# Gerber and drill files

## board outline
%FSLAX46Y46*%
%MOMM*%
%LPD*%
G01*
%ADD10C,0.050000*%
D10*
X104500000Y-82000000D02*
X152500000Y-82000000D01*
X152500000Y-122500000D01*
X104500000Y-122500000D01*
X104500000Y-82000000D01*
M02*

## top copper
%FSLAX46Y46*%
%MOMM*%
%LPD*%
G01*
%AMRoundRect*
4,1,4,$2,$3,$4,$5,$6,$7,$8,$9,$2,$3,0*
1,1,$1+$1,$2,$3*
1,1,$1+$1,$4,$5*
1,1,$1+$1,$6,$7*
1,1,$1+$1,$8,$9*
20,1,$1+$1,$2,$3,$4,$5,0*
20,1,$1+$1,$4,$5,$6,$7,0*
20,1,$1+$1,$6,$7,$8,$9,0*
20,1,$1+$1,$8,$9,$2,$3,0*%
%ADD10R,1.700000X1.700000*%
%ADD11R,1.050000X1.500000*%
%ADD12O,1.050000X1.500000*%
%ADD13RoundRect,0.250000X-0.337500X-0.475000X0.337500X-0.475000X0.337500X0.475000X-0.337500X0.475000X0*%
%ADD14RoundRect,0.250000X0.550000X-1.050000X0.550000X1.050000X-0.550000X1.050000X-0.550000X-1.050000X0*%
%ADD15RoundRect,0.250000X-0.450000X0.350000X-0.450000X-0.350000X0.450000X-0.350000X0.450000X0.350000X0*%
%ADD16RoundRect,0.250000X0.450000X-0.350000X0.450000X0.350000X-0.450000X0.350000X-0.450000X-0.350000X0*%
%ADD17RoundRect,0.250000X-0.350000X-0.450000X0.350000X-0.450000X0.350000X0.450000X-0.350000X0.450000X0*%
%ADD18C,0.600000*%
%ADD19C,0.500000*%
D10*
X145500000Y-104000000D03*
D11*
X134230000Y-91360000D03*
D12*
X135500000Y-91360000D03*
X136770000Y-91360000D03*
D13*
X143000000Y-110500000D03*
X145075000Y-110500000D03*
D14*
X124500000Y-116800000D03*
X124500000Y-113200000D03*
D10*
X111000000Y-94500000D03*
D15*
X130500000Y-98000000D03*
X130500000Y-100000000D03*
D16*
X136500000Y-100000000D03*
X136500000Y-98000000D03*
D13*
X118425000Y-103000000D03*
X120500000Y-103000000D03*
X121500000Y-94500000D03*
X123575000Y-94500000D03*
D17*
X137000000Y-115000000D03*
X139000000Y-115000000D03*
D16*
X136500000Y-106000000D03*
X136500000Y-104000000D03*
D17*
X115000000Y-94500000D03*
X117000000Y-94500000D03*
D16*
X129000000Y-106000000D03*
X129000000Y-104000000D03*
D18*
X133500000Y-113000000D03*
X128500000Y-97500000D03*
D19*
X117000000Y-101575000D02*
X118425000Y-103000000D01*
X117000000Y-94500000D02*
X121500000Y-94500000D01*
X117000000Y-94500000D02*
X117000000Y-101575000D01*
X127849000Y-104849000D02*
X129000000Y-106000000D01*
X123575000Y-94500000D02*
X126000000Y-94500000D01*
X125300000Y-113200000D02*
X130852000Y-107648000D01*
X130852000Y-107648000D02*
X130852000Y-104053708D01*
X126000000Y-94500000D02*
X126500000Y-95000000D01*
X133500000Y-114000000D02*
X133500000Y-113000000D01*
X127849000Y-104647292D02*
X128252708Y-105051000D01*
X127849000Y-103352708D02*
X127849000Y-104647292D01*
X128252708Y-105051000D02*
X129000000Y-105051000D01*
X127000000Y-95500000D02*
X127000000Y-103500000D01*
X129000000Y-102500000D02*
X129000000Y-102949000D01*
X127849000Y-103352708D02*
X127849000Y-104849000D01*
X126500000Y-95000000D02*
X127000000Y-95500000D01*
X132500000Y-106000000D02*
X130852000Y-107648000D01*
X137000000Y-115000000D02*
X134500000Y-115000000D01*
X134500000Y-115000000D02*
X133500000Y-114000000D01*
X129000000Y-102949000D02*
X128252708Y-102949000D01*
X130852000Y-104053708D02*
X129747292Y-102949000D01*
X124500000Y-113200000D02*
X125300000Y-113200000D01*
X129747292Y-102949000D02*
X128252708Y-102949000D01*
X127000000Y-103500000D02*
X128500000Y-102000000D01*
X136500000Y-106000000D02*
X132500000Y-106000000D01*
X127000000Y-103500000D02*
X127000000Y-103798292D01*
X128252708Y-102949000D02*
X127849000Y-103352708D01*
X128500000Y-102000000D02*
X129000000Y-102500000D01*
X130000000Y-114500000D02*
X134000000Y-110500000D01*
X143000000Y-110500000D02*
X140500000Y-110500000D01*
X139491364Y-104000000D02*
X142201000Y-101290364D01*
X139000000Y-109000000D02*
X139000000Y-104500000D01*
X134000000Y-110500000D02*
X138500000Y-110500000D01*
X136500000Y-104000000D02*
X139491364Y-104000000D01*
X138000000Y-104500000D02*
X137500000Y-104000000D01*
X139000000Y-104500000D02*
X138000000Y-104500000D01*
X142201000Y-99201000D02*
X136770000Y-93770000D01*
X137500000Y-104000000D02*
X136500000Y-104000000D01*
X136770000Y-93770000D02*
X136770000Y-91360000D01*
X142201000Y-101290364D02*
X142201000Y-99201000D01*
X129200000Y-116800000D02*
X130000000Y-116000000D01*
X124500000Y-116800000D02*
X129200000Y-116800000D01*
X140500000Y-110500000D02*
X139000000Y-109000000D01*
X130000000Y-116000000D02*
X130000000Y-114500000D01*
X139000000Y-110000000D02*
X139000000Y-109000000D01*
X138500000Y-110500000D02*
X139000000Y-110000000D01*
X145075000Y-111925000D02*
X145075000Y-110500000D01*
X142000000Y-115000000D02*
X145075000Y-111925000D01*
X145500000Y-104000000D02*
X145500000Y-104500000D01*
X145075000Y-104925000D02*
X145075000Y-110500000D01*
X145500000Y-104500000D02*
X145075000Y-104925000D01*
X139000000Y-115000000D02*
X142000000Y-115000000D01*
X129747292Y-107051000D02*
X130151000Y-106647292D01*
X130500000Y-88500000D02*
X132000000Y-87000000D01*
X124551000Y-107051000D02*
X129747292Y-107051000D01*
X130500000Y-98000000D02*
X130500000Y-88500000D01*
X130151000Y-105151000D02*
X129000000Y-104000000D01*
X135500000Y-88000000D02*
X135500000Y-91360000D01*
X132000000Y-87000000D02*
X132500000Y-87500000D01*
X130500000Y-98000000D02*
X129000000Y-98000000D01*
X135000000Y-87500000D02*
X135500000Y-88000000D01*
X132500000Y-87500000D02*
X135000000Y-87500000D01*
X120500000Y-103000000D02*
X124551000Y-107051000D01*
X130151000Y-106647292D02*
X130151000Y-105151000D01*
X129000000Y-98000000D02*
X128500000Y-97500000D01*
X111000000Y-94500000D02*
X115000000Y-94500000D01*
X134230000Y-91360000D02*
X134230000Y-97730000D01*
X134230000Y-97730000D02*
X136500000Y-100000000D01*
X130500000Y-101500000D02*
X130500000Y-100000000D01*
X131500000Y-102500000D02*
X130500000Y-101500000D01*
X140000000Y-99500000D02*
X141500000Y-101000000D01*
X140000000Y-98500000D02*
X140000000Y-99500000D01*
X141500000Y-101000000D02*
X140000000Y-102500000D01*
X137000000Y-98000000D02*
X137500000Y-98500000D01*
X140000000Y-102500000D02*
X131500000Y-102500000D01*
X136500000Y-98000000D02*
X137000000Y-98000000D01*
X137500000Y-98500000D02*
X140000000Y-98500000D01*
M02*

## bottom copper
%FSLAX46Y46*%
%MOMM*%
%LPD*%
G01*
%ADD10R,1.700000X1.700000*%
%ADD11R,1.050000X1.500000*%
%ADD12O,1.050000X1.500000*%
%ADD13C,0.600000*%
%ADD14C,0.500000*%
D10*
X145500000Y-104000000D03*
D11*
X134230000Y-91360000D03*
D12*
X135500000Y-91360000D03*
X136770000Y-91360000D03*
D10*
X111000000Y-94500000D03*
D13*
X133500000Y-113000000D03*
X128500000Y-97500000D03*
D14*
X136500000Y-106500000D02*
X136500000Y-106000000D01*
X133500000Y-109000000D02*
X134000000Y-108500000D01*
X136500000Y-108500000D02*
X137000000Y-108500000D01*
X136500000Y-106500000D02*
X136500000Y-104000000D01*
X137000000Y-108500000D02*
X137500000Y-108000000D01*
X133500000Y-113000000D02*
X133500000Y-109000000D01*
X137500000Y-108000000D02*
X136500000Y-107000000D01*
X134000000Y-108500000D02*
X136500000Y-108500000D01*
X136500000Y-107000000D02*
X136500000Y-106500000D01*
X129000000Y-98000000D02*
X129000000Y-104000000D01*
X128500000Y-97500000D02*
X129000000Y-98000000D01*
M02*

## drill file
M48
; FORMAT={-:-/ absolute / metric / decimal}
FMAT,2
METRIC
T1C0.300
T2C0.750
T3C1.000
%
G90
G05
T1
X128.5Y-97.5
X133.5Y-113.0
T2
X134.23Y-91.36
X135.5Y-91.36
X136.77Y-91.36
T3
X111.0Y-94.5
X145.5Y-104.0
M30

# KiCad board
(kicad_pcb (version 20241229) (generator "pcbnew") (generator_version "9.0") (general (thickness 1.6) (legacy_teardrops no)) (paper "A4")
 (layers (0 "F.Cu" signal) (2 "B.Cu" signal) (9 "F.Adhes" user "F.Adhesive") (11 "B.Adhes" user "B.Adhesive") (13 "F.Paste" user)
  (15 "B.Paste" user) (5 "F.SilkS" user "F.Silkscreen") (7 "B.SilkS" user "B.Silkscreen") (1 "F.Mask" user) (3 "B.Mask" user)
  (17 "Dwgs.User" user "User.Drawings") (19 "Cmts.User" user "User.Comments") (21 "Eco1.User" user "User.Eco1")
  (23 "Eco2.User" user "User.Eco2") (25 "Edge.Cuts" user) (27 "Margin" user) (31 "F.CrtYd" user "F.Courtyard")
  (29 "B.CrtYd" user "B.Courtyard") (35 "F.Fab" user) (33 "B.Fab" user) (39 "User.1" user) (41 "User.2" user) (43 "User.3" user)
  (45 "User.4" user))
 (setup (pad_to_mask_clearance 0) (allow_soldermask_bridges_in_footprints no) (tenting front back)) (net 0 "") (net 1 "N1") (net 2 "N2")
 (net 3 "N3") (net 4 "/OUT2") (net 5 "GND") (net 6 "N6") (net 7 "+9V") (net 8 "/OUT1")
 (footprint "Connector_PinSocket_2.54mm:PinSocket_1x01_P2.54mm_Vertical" (layer "F.Cu") (at 145.5 104)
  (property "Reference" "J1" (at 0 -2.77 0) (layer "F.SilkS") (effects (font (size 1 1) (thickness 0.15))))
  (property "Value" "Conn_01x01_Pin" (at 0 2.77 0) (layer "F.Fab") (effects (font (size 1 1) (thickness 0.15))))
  (pad "1" thru_hole rect (at 0 0) (size 1.7 1.7) (drill 1) (layers "*.Cu" "*.Mask") (remove_unused_layers no) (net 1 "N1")))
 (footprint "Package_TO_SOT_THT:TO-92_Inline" (layer "F.Cu") (at 134.23 91.36)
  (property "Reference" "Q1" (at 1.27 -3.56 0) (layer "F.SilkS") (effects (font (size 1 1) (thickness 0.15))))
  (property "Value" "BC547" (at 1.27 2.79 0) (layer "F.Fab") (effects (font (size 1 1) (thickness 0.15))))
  (pad "1" thru_hole rect (at 0 0) (size 1.05 1.5) (drill 0.75) (layers "*.Cu" "*.Mask") (remove_unused_layers no) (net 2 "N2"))
  (pad "2" thru_hole oval (at 1.27 0) (size 1.05 1.5) (drill 0.75) (layers "*.Cu" "*.Mask") (remove_unused_layers no) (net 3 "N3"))
  (pad "3" thru_hole oval (at 2.54 0) (size 1.05 1.5) (drill 0.75) (layers "*.Cu" "*.Mask") (remove_unused_layers no) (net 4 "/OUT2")))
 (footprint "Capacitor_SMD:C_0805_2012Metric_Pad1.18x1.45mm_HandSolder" (layer "F.Cu") (at 144.0375 110.5)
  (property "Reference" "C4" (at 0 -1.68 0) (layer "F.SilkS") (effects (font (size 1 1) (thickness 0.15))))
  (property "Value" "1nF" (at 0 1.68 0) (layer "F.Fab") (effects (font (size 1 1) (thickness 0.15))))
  (pad "1" smd roundrect (at -1.0375 0) (size 1.175 1.45) (layers "F.Cu" "F.Mask" "F.Paste") (roundrect_rratio 0.212766) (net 4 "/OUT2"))
  (pad "2" smd roundrect (at 1.0375 0) (size 1.175 1.45) (layers "F.Cu" "F.Mask" "F.Paste") (roundrect_rratio 0.212766) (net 1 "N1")))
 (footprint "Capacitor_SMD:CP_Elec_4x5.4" (layer "F.Cu") (at 124.5 115 90)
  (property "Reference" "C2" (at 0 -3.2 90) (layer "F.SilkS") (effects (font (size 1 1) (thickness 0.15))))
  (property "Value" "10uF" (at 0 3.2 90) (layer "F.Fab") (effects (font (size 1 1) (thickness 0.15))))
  (pad "1" smd roundrect (at -1.8 0 90) (size 2.6 1.6) (layers "F.Cu" "F.Mask" "F.Paste") (roundrect_rratio 0.15625) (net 4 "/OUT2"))
  (pad "2" smd roundrect (at 1.8 0 90) (size 2.6 1.6) (layers "F.Cu" "F.Mask" "F.Paste") (roundrect_rratio 0.15625) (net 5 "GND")))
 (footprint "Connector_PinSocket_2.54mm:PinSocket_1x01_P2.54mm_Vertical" (layer "F.Cu") (at 111 94.5)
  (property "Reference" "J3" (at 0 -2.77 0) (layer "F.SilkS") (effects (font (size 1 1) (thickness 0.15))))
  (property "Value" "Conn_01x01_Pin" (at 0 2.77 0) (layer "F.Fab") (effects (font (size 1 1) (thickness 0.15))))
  (pad "1" thru_hole rect (at 0 0) (size 1.7 1.7) (drill 1) (layers "*.Cu" "*.Mask") (remove_unused_layers no) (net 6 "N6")))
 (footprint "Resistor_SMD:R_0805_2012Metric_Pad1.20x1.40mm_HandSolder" (layer "F.Cu") (at 130.5 99 -90)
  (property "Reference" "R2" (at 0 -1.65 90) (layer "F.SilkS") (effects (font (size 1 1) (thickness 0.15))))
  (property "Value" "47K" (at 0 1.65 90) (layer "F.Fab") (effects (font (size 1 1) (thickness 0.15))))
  (pad "1" smd roundrect (at -1 0 270) (size 1.2 1.4) (layers "F.Cu" "F.Mask" "F.Paste") (roundrect_rratio 0.208333) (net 3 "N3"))
  (pad "2" smd roundrect (at 1 0 270) (size 1.2 1.4) (layers "F.Cu" "F.Mask" "F.Paste") (roundrect_rratio 0.208333) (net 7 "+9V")))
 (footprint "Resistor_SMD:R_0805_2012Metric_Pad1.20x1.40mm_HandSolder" (layer "F.Cu") (at 136.5 99 90)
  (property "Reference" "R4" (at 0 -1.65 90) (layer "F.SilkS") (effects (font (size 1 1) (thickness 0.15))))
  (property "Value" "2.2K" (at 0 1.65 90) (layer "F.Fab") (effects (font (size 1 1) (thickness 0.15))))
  (pad "1" smd roundrect (at -1 0 90) (size 1.2 1.4) (layers "F.Cu" "F.Mask" "F.Paste") (roundrect_rratio 0.208333) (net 2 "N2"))
  (pad "2" smd roundrect (at 1 0 90) (size 1.2 1.4) (layers "F.Cu" "F.Mask" "F.Paste") (roundrect_rratio 0.208333) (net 7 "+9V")))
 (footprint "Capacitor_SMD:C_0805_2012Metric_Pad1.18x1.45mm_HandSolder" (layer "F.Cu") (at 119.4625 103)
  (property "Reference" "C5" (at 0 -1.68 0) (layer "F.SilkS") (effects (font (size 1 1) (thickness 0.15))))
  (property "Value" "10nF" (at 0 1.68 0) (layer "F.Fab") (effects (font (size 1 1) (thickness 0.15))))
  (pad "1" smd roundrect (at -1.0375 0) (size 1.175 1.45) (layers "F.Cu" "F.Mask" "F.Paste") (roundrect_rratio 0.212766) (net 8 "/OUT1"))
  (pad "2" smd roundrect (at 1.0375 0) (size 1.175 1.45) (layers "F.Cu" "F.Mask" "F.Paste") (roundrect_rratio 0.212766) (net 3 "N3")))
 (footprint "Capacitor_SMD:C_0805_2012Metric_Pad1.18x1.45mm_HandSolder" (layer "F.Cu") (at 122.5375 94.5)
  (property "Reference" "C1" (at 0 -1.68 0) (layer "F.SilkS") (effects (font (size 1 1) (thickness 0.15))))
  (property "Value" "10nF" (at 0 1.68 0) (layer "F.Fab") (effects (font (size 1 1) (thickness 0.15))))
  (pad "1" smd roundrect (at -1.0375 0) (size 1.175 1.45) (layers "F.Cu" "F.Mask" "F.Paste") (roundrect_rratio 0.212766) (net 8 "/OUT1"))
  (pad "2" smd roundrect (at 1.0375 0) (size 1.175 1.45) (layers "F.Cu" "F.Mask" "F.Paste") (roundrect_rratio 0.212766) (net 5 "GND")))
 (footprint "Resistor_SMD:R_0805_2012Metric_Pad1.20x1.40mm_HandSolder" (layer "F.Cu") (at 138 115)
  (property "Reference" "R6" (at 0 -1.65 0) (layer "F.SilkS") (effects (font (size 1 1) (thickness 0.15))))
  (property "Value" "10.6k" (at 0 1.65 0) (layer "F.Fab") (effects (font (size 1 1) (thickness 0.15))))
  (pad "1" smd roundrect (at -1 0) (size 1.2 1.4) (layers "F.Cu" "F.Mask" "F.Paste") (roundrect_rratio 0.208333) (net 5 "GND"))
  (pad "2" smd roundrect (at 1 0) (size 1.2 1.4) (layers "F.Cu" "F.Mask" "F.Paste") (roundrect_rratio 0.208333) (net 1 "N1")))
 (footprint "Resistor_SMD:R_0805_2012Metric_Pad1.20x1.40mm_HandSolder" (layer "F.Cu") (at 136.5 105 90)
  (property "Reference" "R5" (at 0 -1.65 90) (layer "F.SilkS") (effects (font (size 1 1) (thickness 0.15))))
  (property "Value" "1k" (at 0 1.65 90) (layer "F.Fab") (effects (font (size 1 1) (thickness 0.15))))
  (pad "1" smd roundrect (at -1 0 90) (size 1.2 1.4) (layers "F.Cu" "F.Mask" "F.Paste") (roundrect_rratio 0.208333) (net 5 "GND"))
  (pad "2" smd roundrect (at 1 0 90) (size 1.2 1.4) (layers "F.Cu" "F.Mask" "F.Paste") (roundrect_rratio 0.208333) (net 4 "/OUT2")))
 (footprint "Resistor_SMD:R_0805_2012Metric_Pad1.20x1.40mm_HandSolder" (layer "F.Cu") (at 116 94.5)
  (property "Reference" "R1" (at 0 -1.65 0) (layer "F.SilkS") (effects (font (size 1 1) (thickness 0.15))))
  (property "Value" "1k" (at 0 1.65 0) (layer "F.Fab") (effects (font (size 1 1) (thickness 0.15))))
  (pad "1" smd roundrect (at -1 0) (size 1.2 1.4) (layers "F.Cu" "F.Mask" "F.Paste") (roundrect_rratio 0.208333) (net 6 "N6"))
  (pad "2" smd roundrect (at 1 0) (size 1.2 1.4) (layers "F.Cu" "F.Mask" "F.Paste") (roundrect_rratio 0.208333) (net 8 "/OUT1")))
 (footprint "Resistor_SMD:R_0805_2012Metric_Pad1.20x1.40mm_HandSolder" (layer "F.Cu") (at 129 105 90)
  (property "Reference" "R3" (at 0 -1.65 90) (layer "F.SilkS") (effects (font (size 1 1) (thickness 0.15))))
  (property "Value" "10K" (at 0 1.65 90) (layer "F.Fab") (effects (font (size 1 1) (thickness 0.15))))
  (pad "1" smd roundrect (at -1 0 90) (size 1.2 1.4) (layers "F.Cu" "F.Mask" "F.Paste") (roundrect_rratio 0.208333) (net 5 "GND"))
  (pad "2" smd roundrect (at 1 0 90) (size 1.2 1.4) (layers "F.Cu" "F.Mask" "F.Paste") (roundrect_rratio 0.208333) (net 3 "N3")))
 (gr_rect (start 104.5 82) (end 152.5 122.5) (stroke (width 0.05) (type default)) (fill no) (layer "Edge.Cuts"))
 (segment (start 117 101.575) (end 118.425 103) (width 0.5) (layer "F.Cu") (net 8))
 (segment (start 117 94.5) (end 121.5 94.5) (width 0.5) (layer "F.Cu") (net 8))
 (segment (start 117 94.5) (end 117 101.575) (width 0.5) (layer "F.Cu") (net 8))
 (segment (start 127.849 104.849) (end 129 106) (width 0.5) (layer "F.Cu") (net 5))
 (segment (start 123.575 94.5) (end 126 94.5) (width 0.5) (layer "F.Cu") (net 5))
 (segment (start 125.3 113.2) (end 130.852 107.648) (width 0.5) (layer "F.Cu") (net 5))
 (segment (start 130.852 107.648) (end 130.852 104.053708) (width 0.5) (layer "F.Cu") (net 5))
 (segment (start 126 94.5) (end 126.5 95) (width 0.5) (layer "F.Cu") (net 5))
 (segment (start 133.5 114) (end 133.5 113) (width 0.5) (layer "F.Cu") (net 5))
 (segment (start 127.849 104.647292) (end 128.252708 105.051) (width 0.5) (layer "F.Cu") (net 5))
 (segment (start 127.849 103.352708) (end 127.849 104.647292) (width 0.5) (layer "F.Cu") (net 5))
 (segment (start 128.252708 105.051) (end 129 105.051) (width 0.5) (layer "F.Cu") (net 5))
 (segment (start 127 95.5) (end 127 103.5) (width 0.5) (layer "F.Cu") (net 5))
 (segment (start 129 102.5) (end 129 102.949) (width 0.5) (layer "F.Cu") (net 5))
 (segment (start 127.849 103.352708) (end 127.849 104.849) (width 0.5) (layer "F.Cu") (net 5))
 (segment (start 126.5 95) (end 127 95.5) (width 0.5) (layer "F.Cu") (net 5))
 (segment (start 132.5 106) (end 130.852 107.648) (width 0.5) (layer "F.Cu") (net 5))
 (segment (start 137 115) (end 134.5 115) (width 0.5) (layer "F.Cu") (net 5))
 (segment (start 134.5 115) (end 133.5 114) (width 0.5) (layer "F.Cu") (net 5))
 (segment (start 129 102.949) (end 128.252708 102.949) (width 0.5) (layer "F.Cu") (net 5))
 (segment (start 130.852 104.053708) (end 129.747292 102.949) (width 0.5) (layer "F.Cu") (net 5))
 (segment (start 124.5 113.2) (end 125.3 113.2) (width 0.5) (layer "F.Cu") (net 5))
 (segment (start 129.747292 102.949) (end 128.252708 102.949) (width 0.5) (layer "F.Cu") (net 5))
 (segment (start 127 103.5) (end 128.5 102) (width 0.5) (layer "F.Cu") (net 5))
 (segment (start 136.5 106) (end 132.5 106) (width 0.5) (layer "F.Cu") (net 5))
 (segment (start 127 103.5) (end 127 103.798292) (width 0.5) (layer "F.Cu") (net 5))
 (segment (start 128.252708 102.949) (end 127.849 103.352708) (width 0.5) (layer "F.Cu") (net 5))
 (segment (start 128.5 102) (end 129 102.5) (width 0.5) (layer "F.Cu") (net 5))
 (via (at 133.5 113) (size 0.6) (drill 0.3) (layers "F.Cu" "B.Cu") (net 5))
 (segment (start 136.5 106.5) (end 136.5 106) (width 0.5) (layer "B.Cu") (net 5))
 (segment (start 133.5 109) (end 134 108.5) (width 0.5) (layer "B.Cu") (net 5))
 (segment (start 136.5 108.5) (end 137 108.5) (width 0.5) (layer "B.Cu") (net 5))
 (segment (start 136.5 106.5) (end 136.5 104) (width 0.5) (layer "B.Cu") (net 5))
 (segment (start 137 108.5) (end 137.5 108) (width 0.5) (layer "B.Cu") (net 5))
 (segment (start 133.5 113) (end 133.5 109) (width 0.5) (layer "B.Cu") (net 5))
 (segment (start 137.5 108) (end 136.5 107) (width 0.5) (layer "B.Cu") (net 5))
 (segment (start 134 108.5) (end 136.5 108.5) (width 0.5) (layer "B.Cu") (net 5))
 (segment (start 136.5 107) (end 136.5 106.5) (width 0.5) (layer "B.Cu") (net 5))
 (segment (start 130 114.5) (end 134 110.5) (width 0.5) (layer "F.Cu") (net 4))
 (segment (start 143 110.5) (end 140.5 110.5) (width 0.5) (layer "F.Cu") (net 4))
 (segment (start 139.491364 104) (end 142.201 101.290364) (width 0.5) (layer "F.Cu") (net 4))
 (segment (start 139 109) (end 139 104.5) (width 0.5) (layer "F.Cu") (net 4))
 (segment (start 134 110.5) (end 138.5 110.5) (width 0.5) (layer "F.Cu") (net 4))
 (segment (start 136.5 104) (end 139.491364 104) (width 0.5) (layer "F.Cu") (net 4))
 (segment (start 138 104.5) (end 137.5 104) (width 0.5) (layer "F.Cu") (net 4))
 (segment (start 139 104.5) (end 138 104.5) (width 0.5) (layer "F.Cu") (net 4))
 (segment (start 142.201 99.201) (end 136.77 93.77) (width 0.5) (layer "F.Cu") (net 4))
 (segment (start 137.5 104) (end 136.5 104) (width 0.5) (layer "F.Cu") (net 4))
 (segment (start 136.77 93.77) (end 136.77 91.36) (width 0.5) (layer "F.Cu") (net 4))
 (segment (start 142.201 101.290364) (end 142.201 99.201) (width 0.5) (layer "F.Cu") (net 4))
 (segment (start 129.2 116.8) (end 130 116) (width 0.5) (layer "F.Cu") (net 4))
 (segment (start 124.5 116.8) (end 129.2 116.8) (width 0.5) (layer "F.Cu") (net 4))
 (segment (start 140.5 110.5) (end 139 109) (width 0.5) (layer "F.Cu") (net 4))
 (segment (start 130 116) (end 130 114.5) (width 0.5) (layer "F.Cu") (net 4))
 (segment (start 139 110) (end 139 109) (width 0.5) (layer "F.Cu") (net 4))
 (segment (start 138.5 110.5) (end 139 110) (width 0.5) (layer "F.Cu") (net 4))
 (segment (start 145.075 111.925) (end 145.075 110.5) (width 0.5) (layer "F.Cu") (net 1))
 (segment (start 142 115) (end 145.075 111.925) (width 0.5) (layer "F.Cu") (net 1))
 (segment (start 145.5 104) (end 145.5 104.5) (width 0.5) (layer "F.Cu") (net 1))
 (segment (start 145.075 104.925) (end 145.075 110.5) (width 0.5) (layer "F.Cu") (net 1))
 (segment (start 145.5 104.5) (end 145.075 104.925) (width 0.5) (layer "F.Cu") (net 1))
 (segment (start 139 115) (end 142 115) (width 0.5) (layer "F.Cu") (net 1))
 (segment (start 129.747292 107.051) (end 130.151 106.647292) (width 0.5) (layer "F.Cu") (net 3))
 (segment (start 130.5 88.5) (end 132 87) (width 0.5) (layer "F.Cu") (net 3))
 (segment (start 124.551 107.051) (end 129.747292 107.051) (width 0.5) (layer "F.Cu") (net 3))
 (segment (start 130.5 98) (end 130.5 88.5) (width 0.5) (layer "F.Cu") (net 3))
 (segment (start 130.151 105.151) (end 129 104) (width 0.5) (layer "F.Cu") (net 3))
 (segment (start 135.5 88) (end 135.5 91.36) (width 0.5) (layer "F.Cu") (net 3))
 (segment (start 132 87) (end 132.5 87.5) (width 0.5) (layer "F.Cu") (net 3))
 (segment (start 130.5 98) (end 129 98) (width 0.5) (layer "F.Cu") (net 3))
 (segment (start 135 87.5) (end 135.5 88) (width 0.5) (layer "F.Cu") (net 3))
 (segment (start 132.5 87.5) (end 135 87.5) (width 0.5) (layer "F.Cu") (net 3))
 (segment (start 120.5 103) (end 124.551 107.051) (width 0.5) (layer "F.Cu") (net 3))
 (segment (start 130.151 106.647292) (end 130.151 105.151) (width 0.5) (layer "F.Cu") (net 3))
 (segment (start 129 98) (end 128.5 97.5) (width 0.5) (layer "F.Cu") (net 3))
 (via (at 128.5 97.5) (size 0.6) (drill 0.3) (layers "F.Cu" "B.Cu") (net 3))
 (segment (start 129 98) (end 129 104) (width 0.5) (layer "B.Cu") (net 3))
 (segment (start 128.5 97.5) (end 129 98) (width 0.5) (layer "B.Cu") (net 3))
 (segment (start 111 94.5) (end 115 94.5) (width 0.5) (layer "F.Cu") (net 6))
 (segment (start 134.23 91.36) (end 134.23 97.73) (width 0.5) (layer "F.Cu") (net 2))
 (segment (start 134.23 97.73) (end 136.5 100) (width 0.5) (layer "F.Cu") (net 2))
 (segment (start 130.5 101.5) (end 130.5 100) (width 0.5) (layer "F.Cu") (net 7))
 (segment (start 131.5 102.5) (end 130.5 101.5) (width 0.5) (layer "F.Cu") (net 7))
 (segment (start 140 99.5) (end 141.5 101) (width 0.5) (layer "F.Cu") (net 7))
 (segment (start 140 98.5) (end 140 99.5) (width 0.5) (layer "F.Cu") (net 7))
 (segment (start 141.5 101) (end 140 102.5) (width 0.5) (layer "F.Cu") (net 7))
 (segment (start 137 98) (end 137.5 98.5) (width 0.5) (layer "F.Cu") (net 7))
 (segment (start 140 102.5) (end 131.5 102.5) (width 0.5) (layer "F.Cu") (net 7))
 (segment (start 136.5 98) (end 137 98) (width 0.5) (layer "F.Cu") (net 7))
 (segment (start 137.5 98.5) (end 140 98.5) (width 0.5) (layer "F.Cu") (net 7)))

